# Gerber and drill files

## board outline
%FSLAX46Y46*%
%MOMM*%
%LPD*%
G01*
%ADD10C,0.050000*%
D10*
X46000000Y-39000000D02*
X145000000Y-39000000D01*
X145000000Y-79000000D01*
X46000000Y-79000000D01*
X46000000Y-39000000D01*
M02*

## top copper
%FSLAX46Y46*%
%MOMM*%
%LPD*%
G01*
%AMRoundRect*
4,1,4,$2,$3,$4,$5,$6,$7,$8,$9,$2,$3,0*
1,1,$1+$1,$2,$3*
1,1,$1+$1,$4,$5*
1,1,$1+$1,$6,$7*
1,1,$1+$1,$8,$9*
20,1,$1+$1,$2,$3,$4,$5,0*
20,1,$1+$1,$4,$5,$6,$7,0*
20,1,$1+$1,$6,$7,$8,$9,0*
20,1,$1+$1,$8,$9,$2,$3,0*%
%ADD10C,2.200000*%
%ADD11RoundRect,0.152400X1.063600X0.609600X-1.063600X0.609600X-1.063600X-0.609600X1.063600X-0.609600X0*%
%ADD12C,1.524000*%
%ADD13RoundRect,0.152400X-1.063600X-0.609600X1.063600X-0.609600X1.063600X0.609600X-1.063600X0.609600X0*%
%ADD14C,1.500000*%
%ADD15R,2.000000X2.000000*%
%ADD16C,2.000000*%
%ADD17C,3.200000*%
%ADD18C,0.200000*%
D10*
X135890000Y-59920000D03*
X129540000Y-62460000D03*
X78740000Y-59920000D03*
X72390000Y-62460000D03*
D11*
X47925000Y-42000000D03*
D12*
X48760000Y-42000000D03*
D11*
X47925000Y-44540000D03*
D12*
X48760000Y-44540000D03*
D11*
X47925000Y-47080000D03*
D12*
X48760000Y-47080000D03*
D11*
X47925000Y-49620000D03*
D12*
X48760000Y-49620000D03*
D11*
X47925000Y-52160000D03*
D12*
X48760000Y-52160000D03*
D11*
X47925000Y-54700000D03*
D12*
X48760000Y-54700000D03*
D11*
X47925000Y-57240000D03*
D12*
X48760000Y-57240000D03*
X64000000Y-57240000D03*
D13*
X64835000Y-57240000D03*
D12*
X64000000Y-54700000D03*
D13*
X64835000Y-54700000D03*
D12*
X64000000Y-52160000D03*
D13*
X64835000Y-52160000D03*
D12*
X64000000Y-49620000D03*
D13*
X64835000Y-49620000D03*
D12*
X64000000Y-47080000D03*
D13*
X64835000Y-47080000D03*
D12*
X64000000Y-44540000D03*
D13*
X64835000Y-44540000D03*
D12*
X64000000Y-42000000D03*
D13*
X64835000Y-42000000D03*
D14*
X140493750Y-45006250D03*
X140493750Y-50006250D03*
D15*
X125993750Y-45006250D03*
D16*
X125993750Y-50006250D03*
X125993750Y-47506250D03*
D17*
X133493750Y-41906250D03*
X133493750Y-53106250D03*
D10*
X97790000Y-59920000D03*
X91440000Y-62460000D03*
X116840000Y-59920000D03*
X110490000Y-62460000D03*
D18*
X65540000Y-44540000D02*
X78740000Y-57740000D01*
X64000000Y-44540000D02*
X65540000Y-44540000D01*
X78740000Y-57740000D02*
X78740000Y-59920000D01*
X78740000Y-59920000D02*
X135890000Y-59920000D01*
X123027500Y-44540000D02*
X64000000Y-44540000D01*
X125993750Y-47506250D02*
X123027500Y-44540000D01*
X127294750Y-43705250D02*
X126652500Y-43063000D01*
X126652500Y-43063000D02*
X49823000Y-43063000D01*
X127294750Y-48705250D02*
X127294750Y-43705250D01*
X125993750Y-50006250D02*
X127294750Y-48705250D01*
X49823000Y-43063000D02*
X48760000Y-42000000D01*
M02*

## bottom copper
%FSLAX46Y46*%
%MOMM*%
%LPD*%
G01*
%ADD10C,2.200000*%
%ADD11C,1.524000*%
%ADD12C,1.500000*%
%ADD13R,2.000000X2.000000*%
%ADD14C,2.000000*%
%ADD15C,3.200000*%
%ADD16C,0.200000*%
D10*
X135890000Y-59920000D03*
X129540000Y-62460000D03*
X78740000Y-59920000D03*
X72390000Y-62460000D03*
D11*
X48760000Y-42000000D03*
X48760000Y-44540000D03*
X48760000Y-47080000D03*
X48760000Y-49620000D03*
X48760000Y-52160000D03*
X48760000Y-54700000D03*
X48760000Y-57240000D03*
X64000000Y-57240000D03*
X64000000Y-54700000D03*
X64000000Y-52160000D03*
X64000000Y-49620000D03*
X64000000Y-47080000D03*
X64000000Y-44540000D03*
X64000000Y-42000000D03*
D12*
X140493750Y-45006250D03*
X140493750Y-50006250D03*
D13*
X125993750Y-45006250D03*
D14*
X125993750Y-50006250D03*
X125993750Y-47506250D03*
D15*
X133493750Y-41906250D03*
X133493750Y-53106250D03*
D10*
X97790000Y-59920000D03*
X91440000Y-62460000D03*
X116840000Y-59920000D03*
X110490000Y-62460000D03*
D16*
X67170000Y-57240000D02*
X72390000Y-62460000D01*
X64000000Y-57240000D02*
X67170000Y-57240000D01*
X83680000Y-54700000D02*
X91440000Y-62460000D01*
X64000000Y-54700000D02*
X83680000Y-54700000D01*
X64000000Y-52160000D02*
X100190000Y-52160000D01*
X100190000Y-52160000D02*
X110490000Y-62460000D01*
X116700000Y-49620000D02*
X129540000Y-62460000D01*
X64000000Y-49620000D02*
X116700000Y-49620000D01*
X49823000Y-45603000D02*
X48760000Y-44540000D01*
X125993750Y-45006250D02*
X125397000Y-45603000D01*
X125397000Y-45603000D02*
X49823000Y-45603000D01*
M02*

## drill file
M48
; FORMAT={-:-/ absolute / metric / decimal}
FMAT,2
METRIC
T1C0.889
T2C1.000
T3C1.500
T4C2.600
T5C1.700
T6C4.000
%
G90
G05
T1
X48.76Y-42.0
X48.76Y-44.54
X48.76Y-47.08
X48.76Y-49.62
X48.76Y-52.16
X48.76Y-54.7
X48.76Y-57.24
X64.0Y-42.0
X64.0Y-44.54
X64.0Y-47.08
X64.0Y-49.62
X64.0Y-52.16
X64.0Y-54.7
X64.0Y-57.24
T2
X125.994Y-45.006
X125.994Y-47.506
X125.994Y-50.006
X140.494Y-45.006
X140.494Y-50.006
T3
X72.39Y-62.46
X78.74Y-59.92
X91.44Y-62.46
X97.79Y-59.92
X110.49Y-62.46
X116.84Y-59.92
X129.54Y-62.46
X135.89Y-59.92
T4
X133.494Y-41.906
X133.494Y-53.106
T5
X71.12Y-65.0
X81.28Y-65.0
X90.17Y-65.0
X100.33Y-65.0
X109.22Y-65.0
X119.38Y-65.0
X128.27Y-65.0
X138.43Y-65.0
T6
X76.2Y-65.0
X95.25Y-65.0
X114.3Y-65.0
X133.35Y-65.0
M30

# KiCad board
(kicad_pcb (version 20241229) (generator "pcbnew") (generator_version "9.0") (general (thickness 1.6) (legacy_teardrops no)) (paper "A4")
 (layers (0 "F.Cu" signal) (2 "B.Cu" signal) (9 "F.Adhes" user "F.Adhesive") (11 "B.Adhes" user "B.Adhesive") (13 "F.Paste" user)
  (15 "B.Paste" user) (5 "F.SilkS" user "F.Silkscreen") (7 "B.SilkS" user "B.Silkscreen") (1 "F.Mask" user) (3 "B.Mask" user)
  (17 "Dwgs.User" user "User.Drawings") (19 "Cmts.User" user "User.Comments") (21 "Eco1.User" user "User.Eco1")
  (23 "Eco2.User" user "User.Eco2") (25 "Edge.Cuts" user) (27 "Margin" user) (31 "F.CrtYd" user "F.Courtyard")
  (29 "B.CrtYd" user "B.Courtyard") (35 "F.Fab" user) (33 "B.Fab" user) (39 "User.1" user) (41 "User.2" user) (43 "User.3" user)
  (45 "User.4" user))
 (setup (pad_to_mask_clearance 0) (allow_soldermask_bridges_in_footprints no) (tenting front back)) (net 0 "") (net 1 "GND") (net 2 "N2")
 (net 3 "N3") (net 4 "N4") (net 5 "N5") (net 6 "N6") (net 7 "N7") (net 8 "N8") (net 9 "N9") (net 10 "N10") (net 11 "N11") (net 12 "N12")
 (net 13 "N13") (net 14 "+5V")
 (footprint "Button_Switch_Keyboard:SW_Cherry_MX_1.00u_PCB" (layer "F.Cu") (at 135.89 59.92)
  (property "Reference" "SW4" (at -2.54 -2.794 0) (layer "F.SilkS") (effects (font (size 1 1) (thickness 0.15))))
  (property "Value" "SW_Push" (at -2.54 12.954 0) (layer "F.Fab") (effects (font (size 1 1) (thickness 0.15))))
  (pad "" np_thru_hole circle (at -7.62 5.08) (size 1.7 1.7) (drill 1.7) (layers "*.Cu" "*.Mask"))
  (pad "" np_thru_hole circle (at -2.54 5.08) (size 4 4) (drill 4) (layers "*.Cu" "*.Mask"))
  (pad "" np_thru_hole circle (at 2.54 5.08) (size 1.7 1.7) (drill 1.7) (layers "*.Cu" "*.Mask"))
  (pad "1" thru_hole circle (at 0 0) (size 2.2 2.2) (drill 1.5) (layers "*.Cu" "*.Mask") (remove_unused_layers no) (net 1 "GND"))
  (pad "2" thru_hole circle (at -6.35 2.54) (size 2.2 2.2) (drill 1.5) (layers "*.Cu" "*.Mask") (remove_unused_layers no) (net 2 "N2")))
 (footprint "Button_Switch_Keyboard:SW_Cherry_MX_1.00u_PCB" (layer "F.Cu") (at 78.74 59.92)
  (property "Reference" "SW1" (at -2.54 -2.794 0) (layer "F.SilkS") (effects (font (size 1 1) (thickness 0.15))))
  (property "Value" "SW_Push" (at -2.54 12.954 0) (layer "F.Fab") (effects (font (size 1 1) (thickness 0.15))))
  (pad "" np_thru_hole circle (at -7.62 5.08) (size 1.7 1.7) (drill 1.7) (layers "*.Cu" "*.Mask"))
  (pad "" np_thru_hole circle (at -2.54 5.08) (size 4 4) (drill 4) (layers "*.Cu" "*.Mask"))
  (pad "" np_thru_hole circle (at 2.54 5.08) (size 1.7 1.7) (drill 1.7) (layers "*.Cu" "*.Mask"))
  (pad "1" thru_hole circle (at 0 0) (size 2.2 2.2) (drill 1.5) (layers "*.Cu" "*.Mask") (remove_unused_layers no) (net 1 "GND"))
  (pad "2" thru_hole circle (at -6.35 2.54) (size 2.2 2.2) (drill 1.5) (layers "*.Cu" "*.Mask") (remove_unused_layers no) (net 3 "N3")))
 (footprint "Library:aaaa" (layer "F.Cu") (at 55.52 69.87)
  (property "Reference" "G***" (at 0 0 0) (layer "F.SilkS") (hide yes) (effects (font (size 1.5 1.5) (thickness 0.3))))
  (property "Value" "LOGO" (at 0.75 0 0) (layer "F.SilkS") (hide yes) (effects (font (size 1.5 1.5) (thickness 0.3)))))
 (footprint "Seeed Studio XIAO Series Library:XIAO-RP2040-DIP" (layer "F.Cu") (at 56.38 49.62)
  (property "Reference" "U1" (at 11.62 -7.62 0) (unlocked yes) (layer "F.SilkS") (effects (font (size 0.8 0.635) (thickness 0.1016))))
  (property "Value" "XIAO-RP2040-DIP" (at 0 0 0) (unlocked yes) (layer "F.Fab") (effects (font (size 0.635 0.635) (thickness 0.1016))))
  (pad "1" smd roundrect (at -8.455 -7.62 180) (size 2.432 1.524) (layers "F.Cu" "F.Mask") (roundrect_rratio 0.1) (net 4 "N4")
   (thermal_bridge_angle 45))
  (pad "1" thru_hole circle (at -7.62 -7.62 180) (size 1.524 1.524) (drill 0.889) (layers "*.Cu" "*.Mask") (remove_unused_layers no)
   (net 4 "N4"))
  (pad "2" smd roundrect (at -8.455 -5.08 180) (size 2.432 1.524) (layers "F.Cu" "F.Mask") (roundrect_rratio 0.1) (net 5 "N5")
   (thermal_bridge_angle 45))
  (pad "2" thru_hole circle (at -7.62 -5.08 180) (size 1.524 1.524) (drill 0.889) (layers "*.Cu" "*.Mask") (remove_unused_layers no)
   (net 5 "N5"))
  (pad "3" smd roundrect (at -8.455 -2.54 180) (size 2.432 1.524) (layers "F.Cu" "F.Mask") (roundrect_rratio 0.1) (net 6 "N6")
   (thermal_bridge_angle 45))
  (pad "3" thru_hole circle (at -7.62 -2.54 180) (size 1.524 1.524) (drill 0.889) (layers "*.Cu" "*.Mask") (remove_unused_layers no)
   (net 6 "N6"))
  (pad "4" smd roundrect (at -8.455 0 180) (size 2.432 1.524) (layers "F.Cu" "F.Mask") (roundrect_rratio 0.1) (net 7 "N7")
   (thermal_bridge_angle 45))
  (pad "4" thru_hole circle (at -7.62 0 180) (size 1.524 1.524) (drill 0.889) (layers "*.Cu" "*.Mask") (remove_unused_layers no)
   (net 7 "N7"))
  (pad "5" smd roundrect (at -8.455 2.54 180) (size 2.432 1.524) (layers "F.Cu" "F.Mask") (roundrect_rratio 0.1) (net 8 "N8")
   (thermal_bridge_angle 45))
  (pad "5" thru_hole circle (at -7.62 2.54 180) (size 1.524 1.524) (drill 0.889) (layers "*.Cu" "*.Mask") (remove_unused_layers no)
   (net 8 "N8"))
  (pad "6" smd roundrect (at -8.455 5.08 180) (size 2.432 1.524) (layers "F.Cu" "F.Mask") (roundrect_rratio 0.1) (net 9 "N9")
   (thermal_bridge_angle 45))
  (pad "6" thru_hole circle (at -7.62 5.08 180) (size 1.524 1.524) (drill 0.889) (layers "*.Cu" "*.Mask") (remove_unused_layers no)
   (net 9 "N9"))
  (pad "7" smd roundrect (at -8.455 7.62 180) (size 2.432 1.524) (layers "F.Cu" "F.Mask") (roundrect_rratio 0.1) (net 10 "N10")
   (thermal_bridge_angle 45))
  (pad "7" thru_hole circle (at -7.62 7.62 180) (size 1.524 1.524) (drill 0.889) (layers "*.Cu" "*.Mask") (remove_unused_layers no)
   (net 10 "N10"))
  (pad "8" thru_hole circle (at 7.62 7.62) (size 1.524 1.524) (drill 0.889) (layers "*.Cu" "*.Mask") (remove_unused_layers no) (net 3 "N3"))
  (pad "8" smd roundrect (at 8.455 7.62) (size 2.432 1.524) (layers "F.Cu" "F.Mask") (roundrect_rratio 0.1) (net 3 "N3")
   (thermal_bridge_angle 45))
  (pad "9" thru_hole circle (at 7.62 5.08) (size 1.524 1.524) (drill 0.889) (layers "*.Cu" "*.Mask") (remove_unused_layers no)
   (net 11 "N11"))
  (pad "9" smd roundrect (at 8.455 5.08) (size 2.432 1.524) (layers "F.Cu" "F.Mask") (roundrect_rratio 0.1) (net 11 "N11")
   (thermal_bridge_angle 45))
  (pad "10" thru_hole circle (at 7.62 2.54) (size 1.524 1.524) (drill 0.889) (layers "*.Cu" "*.Mask") (remove_unused_layers no)
   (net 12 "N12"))
  (pad "10" smd roundrect (at 8.455 2.54) (size 2.432 1.524) (layers "F.Cu" "F.Mask") (roundrect_rratio 0.1) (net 12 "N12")
   (thermal_bridge_angle 45))
  (pad "11" thru_hole circle (at 7.62 0) (size 1.524 1.524) (drill 0.889) (layers "*.Cu" "*.Mask") (remove_unused_layers no) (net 2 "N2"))
  (pad "11" smd roundrect (at 8.455 0) (size 2.432 1.524) (layers "F.Cu" "F.Mask") (roundrect_rratio 0.1) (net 2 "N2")
   (thermal_bridge_angle 45))
  (pad "12" thru_hole circle (at 7.62 -2.54) (size 1.524 1.524) (drill 0.889) (layers "*.Cu" "*.Mask") (remove_unused_layers no)
   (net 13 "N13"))
  (pad "12" smd roundrect (at 8.455 -2.54) (size 2.432 1.524) (layers "F.Cu" "F.Mask") (roundrect_rratio 0.1) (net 13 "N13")
   (thermal_bridge_angle 45))
  (pad "13" thru_hole circle (at 7.62 -5.08) (size 1.524 1.524) (drill 0.889) (layers "*.Cu" "*.Mask") (remove_unused_layers no)
   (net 1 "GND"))
  (pad "13" smd roundrect (at 8.455 -5.08) (size 2.432 1.524) (layers "F.Cu" "F.Mask") (roundrect_rratio 0.1) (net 1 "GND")
   (thermal_bridge_angle 45))
  (pad "14" thru_hole circle (at 7.62 -7.62) (size 1.524 1.524) (drill 0.889) (layers "*.Cu" "*.Mask") (remove_unused_layers no)
   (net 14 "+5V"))
  (pad "14" smd roundrect (at 8.455 -7.62) (size 2.432 1.524) (layers "F.Cu" "F.Mask") (roundrect_rratio 0.1) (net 14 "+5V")
   (thermal_bridge_angle 45)))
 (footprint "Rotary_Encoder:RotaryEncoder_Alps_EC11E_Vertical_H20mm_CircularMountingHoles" (layer "F.Cu") (at 125.99375 45.00625)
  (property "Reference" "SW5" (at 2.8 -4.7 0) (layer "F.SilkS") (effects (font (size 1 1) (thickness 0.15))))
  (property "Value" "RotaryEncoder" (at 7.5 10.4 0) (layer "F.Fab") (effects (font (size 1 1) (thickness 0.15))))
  (pad "" thru_hole circle (at 14.5 0) (size 1.5 1.5) (drill 1) (layers "*.Cu" "*.Mask") (remove_unused_layers no))
  (pad "" thru_hole circle (at 14.5 5) (size 1.5 1.5) (drill 1) (layers "*.Cu" "*.Mask") (remove_unused_layers no))
  (pad "A" thru_hole rect (at 0 0) (size 2 2) (drill 1) (layers "*.Cu" "*.Mask") (remove_unused_layers no) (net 5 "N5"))
  (pad "B" thru_hole circle (at 0 5) (size 2 2) (drill 1) (layers "*.Cu" "*.Mask") (remove_unused_layers no) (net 4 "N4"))
  (pad "C" thru_hole circle (at 0 2.5) (size 2 2) (drill 1) (layers "*.Cu" "*.Mask") (remove_unused_layers no) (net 1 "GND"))
  (pad "MP" thru_hole circle (at 7.5 -3.1) (size 3.2 3.2) (drill 2.6) (layers "*.Cu" "*.Mask") (remove_unused_layers no))
  (pad "MP" thru_hole circle (at 7.5 8.1) (size 3.2 3.2) (drill 2.6) (layers "*.Cu" "*.Mask") (remove_unused_layers no)))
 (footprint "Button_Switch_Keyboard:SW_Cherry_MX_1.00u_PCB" (layer "F.Cu") (at 97.79 59.92)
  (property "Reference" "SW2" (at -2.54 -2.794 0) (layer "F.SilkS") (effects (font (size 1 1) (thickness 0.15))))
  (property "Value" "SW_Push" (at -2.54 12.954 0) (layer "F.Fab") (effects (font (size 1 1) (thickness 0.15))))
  (pad "" np_thru_hole circle (at -7.62 5.08) (size 1.7 1.7) (drill 1.7) (layers "*.Cu" "*.Mask"))
  (pad "" np_thru_hole circle (at -2.54 5.08) (size 4 4) (drill 4) (layers "*.Cu" "*.Mask"))
  (pad "" np_thru_hole circle (at 2.54 5.08) (size 1.7 1.7) (drill 1.7) (layers "*.Cu" "*.Mask"))
  (pad "1" thru_hole circle (at 0 0) (size 2.2 2.2) (drill 1.5) (layers "*.Cu" "*.Mask") (remove_unused_layers no) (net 1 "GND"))
  (pad "2" thru_hole circle (at -6.35 2.54) (size 2.2 2.2) (drill 1.5) (layers "*.Cu" "*.Mask") (remove_unused_layers no) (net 11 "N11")))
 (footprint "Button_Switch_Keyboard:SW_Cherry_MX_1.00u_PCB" (layer "F.Cu") (at 116.84 59.92)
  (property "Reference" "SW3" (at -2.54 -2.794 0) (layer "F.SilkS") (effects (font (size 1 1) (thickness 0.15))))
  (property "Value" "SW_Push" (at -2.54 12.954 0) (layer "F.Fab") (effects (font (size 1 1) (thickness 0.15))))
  (pad "" np_thru_hole circle (at -7.62 5.08) (size 1.7 1.7) (drill 1.7) (layers "*.Cu" "*.Mask"))
  (pad "" np_thru_hole circle (at -2.54 5.08) (size 4 4) (drill 4) (layers "*.Cu" "*.Mask"))
  (pad "" np_thru_hole circle (at 2.54 5.08) (size 1.7 1.7) (drill 1.7) (layers "*.Cu" "*.Mask"))
  (pad "1" thru_hole circle (at 0 0) (size 2.2 2.2) (drill 1.5) (layers "*.Cu" "*.Mask") (remove_unused_layers no) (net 1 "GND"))
  (pad "2" thru_hole circle (at -6.35 2.54) (size 2.2 2.2) (drill 1.5) (layers "*.Cu" "*.Mask") (remove_unused_layers no) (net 12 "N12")))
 (gr_rect (start 46 39) (end 145 79) (stroke (width 0.05) (type solid)) (fill no) (layer "Edge.Cuts"))
 (segment (start 65.54 44.54) (end 78.74 57.74) (width 0.2) (layer "F.Cu") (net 1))
 (segment (start 64 44.54) (end 65.54 44.54) (width 0.2) (layer "F.Cu") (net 1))
 (segment (start 78.74 57.74) (end 78.74 59.92) (width 0.2) (layer "F.Cu") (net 1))
 (segment (start 78.74 59.92) (end 135.89 59.92) (width 0.2) (layer "F.Cu") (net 1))
 (segment (start 123.0275 44.54) (end 64 44.54) (width 0.2) (layer "F.Cu") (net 1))
 (segment (start 125.99375 47.50625) (end 123.0275 44.54) (width 0.2) (layer "F.Cu") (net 1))
 (segment (start 67.17 57.24) (end 72.39 62.46) (width 0.2) (layer "B.Cu") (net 3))
 (segment (start 64 57.24) (end 67.17 57.24) (width 0.2) (layer "B.Cu") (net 3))
 (segment (start 83.68 54.7) (end 91.44 62.46) (width 0.2) (layer "B.Cu") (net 11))
 (segment (start 64 54.7) (end 83.68 54.7) (width 0.2) (layer "B.Cu") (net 11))
 (segment (start 64 52.16) (end 100.19 52.16) (width 0.2) (layer "B.Cu") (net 12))
 (segment (start 100.19 52.16) (end 110.49 62.46) (width 0.2) (layer "B.Cu") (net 12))
 (segment (start 116.7 49.62) (end 129.54 62.46) (width 0.2) (layer "B.Cu") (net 2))
 (segment (start 64 49.62) (end 116.7 49.62) (width 0.2) (layer "B.Cu") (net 2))
 (segment (start 49.823 45.603) (end 48.76 44.54) (width 0.2) (layer "B.Cu") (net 5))
 (segment (start 125.99375 45.00625) (end 125.397 45.603) (width 0.2) (layer "B.Cu") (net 5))
 (segment (start 125.397 45.603) (end 49.823 45.603) (width 0.2) (layer "B.Cu") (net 5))
 (segment (start 127.29475 43.70525) (end 126.6525 43.063) (width 0.2) (layer "F.Cu") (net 4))
 (segment (start 126.6525 43.063) (end 49.823 43.063) (width 0.2) (layer "F.Cu") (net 4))
 (segment (start 127.29475 48.70525) (end 127.29475 43.70525) (width 0.2) (layer "F.Cu") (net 4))
 (segment (start 125.99375 50.00625) (end 127.29475 48.70525) (width 0.2) (layer "F.Cu") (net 4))
 (segment (start 49.823 43.063) (end 48.76 42) (width 0.2) (layer "F.Cu") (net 4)))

